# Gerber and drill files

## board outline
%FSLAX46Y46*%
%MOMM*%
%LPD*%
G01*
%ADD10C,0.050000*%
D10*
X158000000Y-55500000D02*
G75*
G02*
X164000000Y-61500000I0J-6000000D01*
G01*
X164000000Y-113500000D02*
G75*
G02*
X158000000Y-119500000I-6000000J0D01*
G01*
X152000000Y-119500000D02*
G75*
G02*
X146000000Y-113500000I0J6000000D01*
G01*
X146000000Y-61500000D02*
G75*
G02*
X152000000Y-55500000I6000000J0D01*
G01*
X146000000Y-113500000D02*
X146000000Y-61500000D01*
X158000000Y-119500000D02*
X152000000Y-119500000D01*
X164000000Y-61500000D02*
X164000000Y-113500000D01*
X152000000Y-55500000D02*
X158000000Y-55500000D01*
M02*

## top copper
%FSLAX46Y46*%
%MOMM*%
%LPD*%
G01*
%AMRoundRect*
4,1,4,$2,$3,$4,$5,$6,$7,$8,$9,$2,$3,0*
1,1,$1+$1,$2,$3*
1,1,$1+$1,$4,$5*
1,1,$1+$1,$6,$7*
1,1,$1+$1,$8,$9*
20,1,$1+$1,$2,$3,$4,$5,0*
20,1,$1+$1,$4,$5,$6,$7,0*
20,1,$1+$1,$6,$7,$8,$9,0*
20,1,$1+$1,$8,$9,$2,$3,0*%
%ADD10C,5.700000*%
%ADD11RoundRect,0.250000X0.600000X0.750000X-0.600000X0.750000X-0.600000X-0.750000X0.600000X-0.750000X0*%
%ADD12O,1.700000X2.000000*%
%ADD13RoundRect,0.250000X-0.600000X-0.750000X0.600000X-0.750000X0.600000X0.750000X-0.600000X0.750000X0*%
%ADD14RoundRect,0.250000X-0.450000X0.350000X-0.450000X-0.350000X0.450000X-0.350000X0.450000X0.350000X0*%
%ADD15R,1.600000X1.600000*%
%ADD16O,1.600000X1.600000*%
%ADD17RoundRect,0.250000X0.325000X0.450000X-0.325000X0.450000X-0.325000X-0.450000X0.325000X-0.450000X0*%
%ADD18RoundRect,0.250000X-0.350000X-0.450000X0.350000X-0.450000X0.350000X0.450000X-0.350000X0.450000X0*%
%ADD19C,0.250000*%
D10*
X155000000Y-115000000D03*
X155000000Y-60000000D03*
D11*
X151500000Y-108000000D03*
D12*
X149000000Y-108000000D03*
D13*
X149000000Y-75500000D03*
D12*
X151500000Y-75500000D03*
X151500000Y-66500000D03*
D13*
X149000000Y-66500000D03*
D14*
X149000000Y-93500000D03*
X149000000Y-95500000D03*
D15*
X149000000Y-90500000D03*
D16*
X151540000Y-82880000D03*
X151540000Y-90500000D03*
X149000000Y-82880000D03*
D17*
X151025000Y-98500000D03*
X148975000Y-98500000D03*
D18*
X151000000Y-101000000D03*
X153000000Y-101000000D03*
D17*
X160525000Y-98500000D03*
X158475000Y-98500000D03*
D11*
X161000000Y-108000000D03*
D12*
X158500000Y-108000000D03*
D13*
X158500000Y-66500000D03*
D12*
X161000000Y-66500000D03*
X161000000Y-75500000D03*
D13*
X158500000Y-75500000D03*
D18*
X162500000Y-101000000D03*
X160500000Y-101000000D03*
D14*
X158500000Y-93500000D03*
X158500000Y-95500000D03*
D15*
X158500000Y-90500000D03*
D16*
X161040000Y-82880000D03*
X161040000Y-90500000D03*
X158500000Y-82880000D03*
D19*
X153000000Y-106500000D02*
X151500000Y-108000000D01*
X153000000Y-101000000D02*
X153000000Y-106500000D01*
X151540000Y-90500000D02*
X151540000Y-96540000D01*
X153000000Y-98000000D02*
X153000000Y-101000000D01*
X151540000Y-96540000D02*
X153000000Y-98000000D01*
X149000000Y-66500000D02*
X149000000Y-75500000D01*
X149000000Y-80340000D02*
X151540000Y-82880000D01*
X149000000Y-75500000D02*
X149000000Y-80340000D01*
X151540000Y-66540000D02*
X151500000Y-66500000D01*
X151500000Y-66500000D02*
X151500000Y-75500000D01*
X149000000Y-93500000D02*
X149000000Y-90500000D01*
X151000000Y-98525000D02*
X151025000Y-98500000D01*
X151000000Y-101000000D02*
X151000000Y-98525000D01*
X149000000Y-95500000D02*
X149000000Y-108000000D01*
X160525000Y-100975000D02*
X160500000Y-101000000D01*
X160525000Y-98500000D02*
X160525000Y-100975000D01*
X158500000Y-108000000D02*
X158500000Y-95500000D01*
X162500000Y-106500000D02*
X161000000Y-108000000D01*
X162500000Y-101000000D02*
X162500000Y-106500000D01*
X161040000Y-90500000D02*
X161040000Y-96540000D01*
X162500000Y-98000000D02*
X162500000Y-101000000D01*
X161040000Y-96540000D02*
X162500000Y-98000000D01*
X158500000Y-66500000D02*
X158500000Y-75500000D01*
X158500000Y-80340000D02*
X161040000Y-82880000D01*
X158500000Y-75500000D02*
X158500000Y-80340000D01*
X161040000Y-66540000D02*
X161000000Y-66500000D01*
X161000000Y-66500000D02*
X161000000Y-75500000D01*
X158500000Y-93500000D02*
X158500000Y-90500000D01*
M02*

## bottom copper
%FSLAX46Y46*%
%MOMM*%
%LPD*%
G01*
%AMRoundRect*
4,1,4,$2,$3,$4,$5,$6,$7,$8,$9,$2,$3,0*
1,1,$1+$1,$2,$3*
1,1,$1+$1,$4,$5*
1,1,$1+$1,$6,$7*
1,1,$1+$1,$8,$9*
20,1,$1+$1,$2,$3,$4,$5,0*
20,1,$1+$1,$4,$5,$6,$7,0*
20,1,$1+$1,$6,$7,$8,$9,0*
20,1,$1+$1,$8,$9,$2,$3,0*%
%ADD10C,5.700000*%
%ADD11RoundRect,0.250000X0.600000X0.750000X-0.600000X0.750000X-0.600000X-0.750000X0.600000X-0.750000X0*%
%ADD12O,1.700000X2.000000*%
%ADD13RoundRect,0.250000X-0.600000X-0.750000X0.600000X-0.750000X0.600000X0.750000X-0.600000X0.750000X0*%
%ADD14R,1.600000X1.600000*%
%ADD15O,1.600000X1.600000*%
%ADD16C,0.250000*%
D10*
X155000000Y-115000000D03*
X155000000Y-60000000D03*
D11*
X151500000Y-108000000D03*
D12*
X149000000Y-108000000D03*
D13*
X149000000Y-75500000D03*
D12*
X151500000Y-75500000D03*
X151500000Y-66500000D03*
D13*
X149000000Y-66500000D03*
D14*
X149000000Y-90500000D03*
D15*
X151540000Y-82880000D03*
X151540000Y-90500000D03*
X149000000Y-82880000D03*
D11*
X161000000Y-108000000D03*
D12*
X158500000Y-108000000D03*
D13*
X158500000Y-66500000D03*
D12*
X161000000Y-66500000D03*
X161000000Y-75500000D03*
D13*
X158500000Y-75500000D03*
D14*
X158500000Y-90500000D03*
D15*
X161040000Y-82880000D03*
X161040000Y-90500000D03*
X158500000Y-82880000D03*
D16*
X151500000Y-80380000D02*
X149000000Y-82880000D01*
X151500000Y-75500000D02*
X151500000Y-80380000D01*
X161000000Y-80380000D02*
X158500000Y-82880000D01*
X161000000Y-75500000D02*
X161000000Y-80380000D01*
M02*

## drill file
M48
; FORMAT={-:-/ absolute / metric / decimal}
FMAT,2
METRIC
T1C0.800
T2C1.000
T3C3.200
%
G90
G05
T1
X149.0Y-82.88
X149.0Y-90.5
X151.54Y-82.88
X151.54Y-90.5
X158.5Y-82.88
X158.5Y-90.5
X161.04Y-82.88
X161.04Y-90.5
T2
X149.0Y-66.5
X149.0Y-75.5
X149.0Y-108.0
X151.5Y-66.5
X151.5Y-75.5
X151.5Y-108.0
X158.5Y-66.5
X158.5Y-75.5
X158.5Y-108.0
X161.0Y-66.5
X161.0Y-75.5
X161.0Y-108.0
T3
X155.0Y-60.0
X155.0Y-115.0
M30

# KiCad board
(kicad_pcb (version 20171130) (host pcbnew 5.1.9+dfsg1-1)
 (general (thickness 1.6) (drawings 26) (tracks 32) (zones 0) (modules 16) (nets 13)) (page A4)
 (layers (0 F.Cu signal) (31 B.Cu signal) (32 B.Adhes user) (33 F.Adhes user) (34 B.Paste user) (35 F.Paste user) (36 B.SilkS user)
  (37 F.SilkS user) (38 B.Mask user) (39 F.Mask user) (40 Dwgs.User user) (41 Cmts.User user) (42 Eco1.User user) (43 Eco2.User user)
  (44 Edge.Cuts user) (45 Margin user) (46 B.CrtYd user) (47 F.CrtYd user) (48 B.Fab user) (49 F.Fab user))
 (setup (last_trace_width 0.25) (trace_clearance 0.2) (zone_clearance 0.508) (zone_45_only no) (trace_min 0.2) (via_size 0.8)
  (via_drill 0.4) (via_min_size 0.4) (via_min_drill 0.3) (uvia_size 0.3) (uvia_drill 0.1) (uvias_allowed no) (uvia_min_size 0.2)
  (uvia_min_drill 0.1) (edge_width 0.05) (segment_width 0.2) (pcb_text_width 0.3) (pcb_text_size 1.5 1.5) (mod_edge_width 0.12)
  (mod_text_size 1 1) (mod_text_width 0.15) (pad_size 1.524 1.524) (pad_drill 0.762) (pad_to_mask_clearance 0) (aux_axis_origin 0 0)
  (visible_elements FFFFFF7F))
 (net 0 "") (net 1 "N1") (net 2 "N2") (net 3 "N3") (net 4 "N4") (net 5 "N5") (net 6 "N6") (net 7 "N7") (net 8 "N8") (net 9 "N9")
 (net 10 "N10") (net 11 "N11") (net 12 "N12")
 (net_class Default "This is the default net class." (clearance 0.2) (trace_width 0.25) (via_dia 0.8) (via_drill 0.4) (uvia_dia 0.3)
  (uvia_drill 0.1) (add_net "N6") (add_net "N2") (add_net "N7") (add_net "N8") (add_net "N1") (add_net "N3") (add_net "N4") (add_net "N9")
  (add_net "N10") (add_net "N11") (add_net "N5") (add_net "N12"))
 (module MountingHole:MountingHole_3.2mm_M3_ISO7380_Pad (layer F.Cu) (at 155 115)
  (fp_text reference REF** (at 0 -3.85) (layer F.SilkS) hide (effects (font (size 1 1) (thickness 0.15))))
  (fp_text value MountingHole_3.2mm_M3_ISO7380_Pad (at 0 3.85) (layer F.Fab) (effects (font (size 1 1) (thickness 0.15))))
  (pad 1 thru_hole circle (at 0 0) (size 5.7 5.7) (drill 3.2) (layers *.Cu *.Mask)))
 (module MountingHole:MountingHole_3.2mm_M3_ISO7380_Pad (layer F.Cu) (at 155 60)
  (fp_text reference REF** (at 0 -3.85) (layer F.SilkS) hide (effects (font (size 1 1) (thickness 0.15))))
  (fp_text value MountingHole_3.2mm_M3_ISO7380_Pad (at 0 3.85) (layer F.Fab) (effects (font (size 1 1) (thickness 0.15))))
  (pad 1 thru_hole circle (at 0 0) (size 5.7 5.7) (drill 3.2) (layers *.Cu *.Mask)))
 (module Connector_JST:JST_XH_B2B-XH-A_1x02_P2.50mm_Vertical (layer F.Cu) (at 151.5 108 180)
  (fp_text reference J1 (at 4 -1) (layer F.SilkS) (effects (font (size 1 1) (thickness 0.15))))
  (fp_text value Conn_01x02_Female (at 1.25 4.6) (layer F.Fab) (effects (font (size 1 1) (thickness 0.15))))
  (pad 1 thru_hole roundrect (at 0 0 180) (size 1.7 2) (drill 1) (layers *.Cu *.Mask) (roundrect_rratio 0.147059) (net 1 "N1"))
  (pad 2 thru_hole oval (at 2.5 0 180) (size 1.7 2) (drill 1) (layers *.Cu *.Mask) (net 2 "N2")))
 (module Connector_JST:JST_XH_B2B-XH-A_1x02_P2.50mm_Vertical (layer F.Cu) (at 149 75.5)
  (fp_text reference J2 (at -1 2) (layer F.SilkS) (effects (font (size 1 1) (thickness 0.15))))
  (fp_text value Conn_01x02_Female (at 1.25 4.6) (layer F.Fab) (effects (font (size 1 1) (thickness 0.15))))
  (pad 1 thru_hole roundrect (at 0 0) (size 1.7 2) (drill 1) (layers *.Cu *.Mask) (roundrect_rratio 0.147059) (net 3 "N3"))
  (pad 2 thru_hole oval (at 2.5 0) (size 1.7 2) (drill 1) (layers *.Cu *.Mask) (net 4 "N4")))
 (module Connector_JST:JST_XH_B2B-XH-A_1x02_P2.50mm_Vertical (layer F.Cu) (at 149 66.5)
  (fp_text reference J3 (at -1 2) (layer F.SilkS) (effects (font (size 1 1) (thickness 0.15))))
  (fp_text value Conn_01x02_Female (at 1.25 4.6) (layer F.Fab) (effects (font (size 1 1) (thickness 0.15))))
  (pad 2 thru_hole oval (at 2.5 0) (size 1.7 2) (drill 1) (layers *.Cu *.Mask) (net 4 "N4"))
  (pad 1 thru_hole roundrect (at 0 0) (size 1.7 2) (drill 1) (layers *.Cu *.Mask) (roundrect_rratio 0.147059) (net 3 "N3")))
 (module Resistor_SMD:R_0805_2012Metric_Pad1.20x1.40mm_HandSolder (layer F.Cu) (at 149 94.5 270)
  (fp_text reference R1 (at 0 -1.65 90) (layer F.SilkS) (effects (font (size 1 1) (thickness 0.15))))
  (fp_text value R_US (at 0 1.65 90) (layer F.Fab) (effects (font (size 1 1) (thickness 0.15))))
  (pad 1 smd roundrect (at -1 0 270) (size 1.2 1.4) (layers F.Cu F.Paste F.Mask) (roundrect_rratio 0.208333) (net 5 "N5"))
  (pad 2 smd roundrect (at 1 0 270) (size 1.2 1.4) (layers F.Cu F.Paste F.Mask) (roundrect_rratio 0.208333) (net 2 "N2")))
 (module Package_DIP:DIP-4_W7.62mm (layer F.Cu) (at 149 90.5 90)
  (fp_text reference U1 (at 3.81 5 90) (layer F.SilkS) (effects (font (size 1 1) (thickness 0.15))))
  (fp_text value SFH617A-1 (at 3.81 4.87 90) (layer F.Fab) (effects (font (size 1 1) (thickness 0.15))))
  (pad 1 thru_hole rect (at 0 0 90) (size 1.6 1.6) (drill 0.8) (layers *.Cu *.Mask) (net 5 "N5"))
  (pad 3 thru_hole oval (at 7.62 2.54 90) (size 1.6 1.6) (drill 0.8) (layers *.Cu *.Mask) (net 3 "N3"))
  (pad 2 thru_hole oval (at 0 2.54 90) (size 1.6 1.6) (drill 0.8) (layers *.Cu *.Mask) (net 1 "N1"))
  (pad 4 thru_hole oval (at 7.62 0 90) (size 1.6 1.6) (drill 0.8) (layers *.Cu *.Mask) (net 4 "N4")))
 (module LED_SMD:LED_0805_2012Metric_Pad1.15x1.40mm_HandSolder (layer F.Cu) (at 150 98.5 180)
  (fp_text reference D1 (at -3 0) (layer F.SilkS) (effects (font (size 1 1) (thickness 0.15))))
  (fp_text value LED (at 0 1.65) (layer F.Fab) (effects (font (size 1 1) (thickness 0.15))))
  (pad 1 smd roundrect (at -1.025 0 180) (size 1.15 1.4) (layers F.Cu F.Paste F.Mask) (roundrect_rratio 0.217391) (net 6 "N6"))
  (pad 2 smd roundrect (at 1.025 0 180) (size 1.15 1.4) (layers F.Cu F.Paste F.Mask) (roundrect_rratio 0.217391) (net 2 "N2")))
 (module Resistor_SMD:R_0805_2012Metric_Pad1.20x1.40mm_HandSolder (layer F.Cu) (at 152 101)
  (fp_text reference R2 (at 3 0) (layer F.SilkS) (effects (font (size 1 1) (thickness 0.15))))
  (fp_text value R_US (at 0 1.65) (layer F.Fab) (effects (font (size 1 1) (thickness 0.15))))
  (pad 1 smd roundrect (at -1 0) (size 1.2 1.4) (layers F.Cu F.Paste F.Mask) (roundrect_rratio 0.208333) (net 6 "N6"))
  (pad 2 smd roundrect (at 1 0) (size 1.2 1.4) (layers F.Cu F.Paste F.Mask) (roundrect_rratio 0.208333) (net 1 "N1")))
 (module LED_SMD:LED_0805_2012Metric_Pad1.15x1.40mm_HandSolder (layer F.Cu) (at 159.5 98.5 180)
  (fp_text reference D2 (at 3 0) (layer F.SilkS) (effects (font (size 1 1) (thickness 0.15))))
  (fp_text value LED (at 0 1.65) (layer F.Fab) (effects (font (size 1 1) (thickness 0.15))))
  (pad 1 smd roundrect (at -1.025 0 180) (size 1.15 1.4) (layers F.Cu F.Paste F.Mask) (roundrect_rratio 0.217391) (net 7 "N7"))
  (pad 2 smd roundrect (at 1.025 0 180) (size 1.15 1.4) (layers F.Cu F.Paste F.Mask) (roundrect_rratio 0.217391) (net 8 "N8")))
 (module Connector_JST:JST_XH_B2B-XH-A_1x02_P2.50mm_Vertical (layer F.Cu) (at 161 108 180)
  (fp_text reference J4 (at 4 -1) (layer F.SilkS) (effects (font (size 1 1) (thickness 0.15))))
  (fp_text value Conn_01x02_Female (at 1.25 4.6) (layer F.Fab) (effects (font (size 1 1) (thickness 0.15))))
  (pad 1 thru_hole roundrect (at 0 0 180) (size 1.7 2) (drill 1) (layers *.Cu *.Mask) (roundrect_rratio 0.147059) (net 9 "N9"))
  (pad 2 thru_hole oval (at 2.5 0 180) (size 1.7 2) (drill 1) (layers *.Cu *.Mask) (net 8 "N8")))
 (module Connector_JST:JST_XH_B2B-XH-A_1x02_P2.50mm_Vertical (layer F.Cu) (at 158.5 66.5)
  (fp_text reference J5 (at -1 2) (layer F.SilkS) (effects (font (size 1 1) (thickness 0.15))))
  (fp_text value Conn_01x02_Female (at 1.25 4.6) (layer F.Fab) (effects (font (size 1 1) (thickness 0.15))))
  (pad 1 thru_hole roundrect (at 0 0) (size 1.7 2) (drill 1) (layers *.Cu *.Mask) (roundrect_rratio 0.147059) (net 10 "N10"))
  (pad 2 thru_hole oval (at 2.5 0) (size 1.7 2) (drill 1) (layers *.Cu *.Mask) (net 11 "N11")))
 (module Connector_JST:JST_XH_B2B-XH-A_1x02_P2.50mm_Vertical (layer F.Cu) (at 158.5 75.5)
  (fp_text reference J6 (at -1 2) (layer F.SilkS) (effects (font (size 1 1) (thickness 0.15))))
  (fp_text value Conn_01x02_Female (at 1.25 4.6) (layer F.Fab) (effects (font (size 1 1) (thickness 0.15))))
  (pad 2 thru_hole oval (at 2.5 0) (size 1.7 2) (drill 1) (layers *.Cu *.Mask) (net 11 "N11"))
  (pad 1 thru_hole roundrect (at 0 0) (size 1.7 2) (drill 1) (layers *.Cu *.Mask) (roundrect_rratio 0.147059) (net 10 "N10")))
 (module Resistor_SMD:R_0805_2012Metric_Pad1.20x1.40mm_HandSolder (layer F.Cu) (at 161.5 101)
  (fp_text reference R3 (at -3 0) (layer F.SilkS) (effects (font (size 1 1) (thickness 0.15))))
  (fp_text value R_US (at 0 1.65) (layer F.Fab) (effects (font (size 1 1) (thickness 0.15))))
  (pad 2 smd roundrect (at 1 0) (size 1.2 1.4) (layers F.Cu F.Paste F.Mask) (roundrect_rratio 0.208333) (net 9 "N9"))
  (pad 1 smd roundrect (at -1 0) (size 1.2 1.4) (layers F.Cu F.Paste F.Mask) (roundrect_rratio 0.208333) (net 7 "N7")))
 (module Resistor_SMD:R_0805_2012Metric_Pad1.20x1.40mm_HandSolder (layer F.Cu) (at 158.5 94.5 270)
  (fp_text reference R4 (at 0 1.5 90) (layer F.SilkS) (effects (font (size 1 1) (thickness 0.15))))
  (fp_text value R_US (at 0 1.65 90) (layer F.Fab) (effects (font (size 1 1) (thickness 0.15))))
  (pad 1 smd roundrect (at -1 0 270) (size 1.2 1.4) (layers F.Cu F.Paste F.Mask) (roundrect_rratio 0.208333) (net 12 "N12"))
  (pad 2 smd roundrect (at 1 0 270) (size 1.2 1.4) (layers F.Cu F.Paste F.Mask) (roundrect_rratio 0.208333) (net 8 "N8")))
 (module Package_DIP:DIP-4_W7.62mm (layer F.Cu) (at 158.5 90.5 90)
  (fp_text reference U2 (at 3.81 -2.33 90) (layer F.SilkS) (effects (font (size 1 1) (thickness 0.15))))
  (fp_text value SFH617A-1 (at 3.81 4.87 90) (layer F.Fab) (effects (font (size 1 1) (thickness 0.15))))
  (pad 1 thru_hole rect (at 0 0 90) (size 1.6 1.6) (drill 0.8) (layers *.Cu *.Mask) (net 12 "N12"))
  (pad 3 thru_hole oval (at 7.62 2.54 90) (size 1.6 1.6) (drill 0.8) (layers *.Cu *.Mask) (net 10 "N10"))
  (pad 2 thru_hole oval (at 0 2.54 90) (size 1.6 1.6) (drill 0.8) (layers *.Cu *.Mask) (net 9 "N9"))
  (pad 4 thru_hole oval (at 7.62 0 90) (size 1.6 1.6) (drill 0.8) (layers *.Cu *.Mask) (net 11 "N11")))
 (gr_arc (start 158 61.5) (end 164 61.5) (angle -90) (layer Edge.Cuts) (width 0.05))
 (gr_arc (start 158 113.5) (end 158 119.5) (angle -90) (layer Edge.Cuts) (width 0.05))
 (gr_arc (start 152 113.5) (end 146 113.5) (angle -90) (layer Edge.Cuts) (width 0.05))
 (gr_arc (start 152 61.5) (end 152 55.5) (angle -90) (layer Edge.Cuts) (width 0.05))
 (gr_line (start 146 113.5) (end 146 61.5) (layer Edge.Cuts) (width 0.05))
 (gr_line (start 158 119.5) (end 152 119.5) (layer Edge.Cuts) (width 0.05))
 (gr_line (start 164 61.5) (end 164 113.5) (layer Edge.Cuts) (width 0.05))
 (gr_line (start 152 55.5) (end 158 55.5) (layer Edge.Cuts) (width 0.05))
 (segment (start 153 106.5) (end 151.5 108) (width 0.25) (layer F.Cu) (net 1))
 (segment (start 153 101) (end 153 106.5) (width 0.25) (layer F.Cu) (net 1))
 (segment (start 151.54 90.5) (end 151.54 96.54) (width 0.25) (layer F.Cu) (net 1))
 (segment (start 153 98) (end 153 101) (width 0.25) (layer F.Cu) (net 1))
 (segment (start 151.54 96.54) (end 153 98) (width 0.25) (layer F.Cu) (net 1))
 (segment (start 149 66.5) (end 149 75.5) (width 0.25) (layer F.Cu) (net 3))
 (segment (start 149 80.34) (end 151.54 82.88) (width 0.25) (layer F.Cu) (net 3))
 (segment (start 149 75.5) (end 149 80.34) (width 0.25) (layer F.Cu) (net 3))
 (segment (start 151.54 66.54) (end 151.5 66.5) (width 0.25) (layer F.Cu) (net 4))
 (segment (start 151.5 66.5) (end 151.5 75.5) (width 0.25) (layer F.Cu) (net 4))
 (segment (start 151.5 80.38) (end 149 82.88) (width 0.25) (layer B.Cu) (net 4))
 (segment (start 151.5 75.5) (end 151.5 80.38) (width 0.25) (layer B.Cu) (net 4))
 (segment (start 149 93.5) (end 149 90.5) (width 0.25) (layer F.Cu) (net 5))
 (segment (start 151 98.525) (end 151.025 98.5) (width 0.25) (layer F.Cu) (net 6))
 (segment (start 151 101) (end 151 98.525) (width 0.25) (layer F.Cu) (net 6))
 (segment (start 149 95.5) (end 149 108) (width 0.25) (layer F.Cu) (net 2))
 (segment (start 160.525 100.975) (end 160.5 101) (width 0.25) (layer F.Cu) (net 7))
 (segment (start 160.525 98.5) (end 160.525 100.975) (width 0.25) (layer F.Cu) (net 7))
 (segment (start 158.5 108) (end 158.5 95.5) (width 0.25) (layer F.Cu) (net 8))
 (segment (start 162.5 106.5) (end 161 108) (width 0.25) (layer F.Cu) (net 9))
 (segment (start 162.5 101) (end 162.5 106.5) (width 0.25) (layer F.Cu) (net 9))
 (segment (start 161.04 90.5) (end 161.04 96.54) (width 0.25) (layer F.Cu) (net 9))
 (segment (start 162.5 98) (end 162.5 101) (width 0.25) (layer F.Cu) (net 9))
 (segment (start 161.04 96.54) (end 162.5 98) (width 0.25) (layer F.Cu) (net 9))
 (segment (start 158.5 66.5) (end 158.5 75.5) (width 0.25) (layer F.Cu) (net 10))
 (segment (start 158.5 80.34) (end 161.04 82.88) (width 0.25) (layer F.Cu) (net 10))
 (segment (start 158.5 75.5) (end 158.5 80.34) (width 0.25) (layer F.Cu) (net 10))
 (segment (start 161.04 66.54) (end 161 66.5) (width 0.25) (layer F.Cu) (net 11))
 (segment (start 161 66.5) (end 161 75.5) (width 0.25) (layer F.Cu) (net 11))
 (segment (start 161 80.38) (end 158.5 82.88) (width 0.25) (layer B.Cu) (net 11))
 (segment (start 161 75.5) (end 161 80.38) (width 0.25) (layer B.Cu) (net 11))
 (segment (start 158.5 93.5) (end 158.5 90.5) (width 0.25) (layer F.Cu) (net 12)))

